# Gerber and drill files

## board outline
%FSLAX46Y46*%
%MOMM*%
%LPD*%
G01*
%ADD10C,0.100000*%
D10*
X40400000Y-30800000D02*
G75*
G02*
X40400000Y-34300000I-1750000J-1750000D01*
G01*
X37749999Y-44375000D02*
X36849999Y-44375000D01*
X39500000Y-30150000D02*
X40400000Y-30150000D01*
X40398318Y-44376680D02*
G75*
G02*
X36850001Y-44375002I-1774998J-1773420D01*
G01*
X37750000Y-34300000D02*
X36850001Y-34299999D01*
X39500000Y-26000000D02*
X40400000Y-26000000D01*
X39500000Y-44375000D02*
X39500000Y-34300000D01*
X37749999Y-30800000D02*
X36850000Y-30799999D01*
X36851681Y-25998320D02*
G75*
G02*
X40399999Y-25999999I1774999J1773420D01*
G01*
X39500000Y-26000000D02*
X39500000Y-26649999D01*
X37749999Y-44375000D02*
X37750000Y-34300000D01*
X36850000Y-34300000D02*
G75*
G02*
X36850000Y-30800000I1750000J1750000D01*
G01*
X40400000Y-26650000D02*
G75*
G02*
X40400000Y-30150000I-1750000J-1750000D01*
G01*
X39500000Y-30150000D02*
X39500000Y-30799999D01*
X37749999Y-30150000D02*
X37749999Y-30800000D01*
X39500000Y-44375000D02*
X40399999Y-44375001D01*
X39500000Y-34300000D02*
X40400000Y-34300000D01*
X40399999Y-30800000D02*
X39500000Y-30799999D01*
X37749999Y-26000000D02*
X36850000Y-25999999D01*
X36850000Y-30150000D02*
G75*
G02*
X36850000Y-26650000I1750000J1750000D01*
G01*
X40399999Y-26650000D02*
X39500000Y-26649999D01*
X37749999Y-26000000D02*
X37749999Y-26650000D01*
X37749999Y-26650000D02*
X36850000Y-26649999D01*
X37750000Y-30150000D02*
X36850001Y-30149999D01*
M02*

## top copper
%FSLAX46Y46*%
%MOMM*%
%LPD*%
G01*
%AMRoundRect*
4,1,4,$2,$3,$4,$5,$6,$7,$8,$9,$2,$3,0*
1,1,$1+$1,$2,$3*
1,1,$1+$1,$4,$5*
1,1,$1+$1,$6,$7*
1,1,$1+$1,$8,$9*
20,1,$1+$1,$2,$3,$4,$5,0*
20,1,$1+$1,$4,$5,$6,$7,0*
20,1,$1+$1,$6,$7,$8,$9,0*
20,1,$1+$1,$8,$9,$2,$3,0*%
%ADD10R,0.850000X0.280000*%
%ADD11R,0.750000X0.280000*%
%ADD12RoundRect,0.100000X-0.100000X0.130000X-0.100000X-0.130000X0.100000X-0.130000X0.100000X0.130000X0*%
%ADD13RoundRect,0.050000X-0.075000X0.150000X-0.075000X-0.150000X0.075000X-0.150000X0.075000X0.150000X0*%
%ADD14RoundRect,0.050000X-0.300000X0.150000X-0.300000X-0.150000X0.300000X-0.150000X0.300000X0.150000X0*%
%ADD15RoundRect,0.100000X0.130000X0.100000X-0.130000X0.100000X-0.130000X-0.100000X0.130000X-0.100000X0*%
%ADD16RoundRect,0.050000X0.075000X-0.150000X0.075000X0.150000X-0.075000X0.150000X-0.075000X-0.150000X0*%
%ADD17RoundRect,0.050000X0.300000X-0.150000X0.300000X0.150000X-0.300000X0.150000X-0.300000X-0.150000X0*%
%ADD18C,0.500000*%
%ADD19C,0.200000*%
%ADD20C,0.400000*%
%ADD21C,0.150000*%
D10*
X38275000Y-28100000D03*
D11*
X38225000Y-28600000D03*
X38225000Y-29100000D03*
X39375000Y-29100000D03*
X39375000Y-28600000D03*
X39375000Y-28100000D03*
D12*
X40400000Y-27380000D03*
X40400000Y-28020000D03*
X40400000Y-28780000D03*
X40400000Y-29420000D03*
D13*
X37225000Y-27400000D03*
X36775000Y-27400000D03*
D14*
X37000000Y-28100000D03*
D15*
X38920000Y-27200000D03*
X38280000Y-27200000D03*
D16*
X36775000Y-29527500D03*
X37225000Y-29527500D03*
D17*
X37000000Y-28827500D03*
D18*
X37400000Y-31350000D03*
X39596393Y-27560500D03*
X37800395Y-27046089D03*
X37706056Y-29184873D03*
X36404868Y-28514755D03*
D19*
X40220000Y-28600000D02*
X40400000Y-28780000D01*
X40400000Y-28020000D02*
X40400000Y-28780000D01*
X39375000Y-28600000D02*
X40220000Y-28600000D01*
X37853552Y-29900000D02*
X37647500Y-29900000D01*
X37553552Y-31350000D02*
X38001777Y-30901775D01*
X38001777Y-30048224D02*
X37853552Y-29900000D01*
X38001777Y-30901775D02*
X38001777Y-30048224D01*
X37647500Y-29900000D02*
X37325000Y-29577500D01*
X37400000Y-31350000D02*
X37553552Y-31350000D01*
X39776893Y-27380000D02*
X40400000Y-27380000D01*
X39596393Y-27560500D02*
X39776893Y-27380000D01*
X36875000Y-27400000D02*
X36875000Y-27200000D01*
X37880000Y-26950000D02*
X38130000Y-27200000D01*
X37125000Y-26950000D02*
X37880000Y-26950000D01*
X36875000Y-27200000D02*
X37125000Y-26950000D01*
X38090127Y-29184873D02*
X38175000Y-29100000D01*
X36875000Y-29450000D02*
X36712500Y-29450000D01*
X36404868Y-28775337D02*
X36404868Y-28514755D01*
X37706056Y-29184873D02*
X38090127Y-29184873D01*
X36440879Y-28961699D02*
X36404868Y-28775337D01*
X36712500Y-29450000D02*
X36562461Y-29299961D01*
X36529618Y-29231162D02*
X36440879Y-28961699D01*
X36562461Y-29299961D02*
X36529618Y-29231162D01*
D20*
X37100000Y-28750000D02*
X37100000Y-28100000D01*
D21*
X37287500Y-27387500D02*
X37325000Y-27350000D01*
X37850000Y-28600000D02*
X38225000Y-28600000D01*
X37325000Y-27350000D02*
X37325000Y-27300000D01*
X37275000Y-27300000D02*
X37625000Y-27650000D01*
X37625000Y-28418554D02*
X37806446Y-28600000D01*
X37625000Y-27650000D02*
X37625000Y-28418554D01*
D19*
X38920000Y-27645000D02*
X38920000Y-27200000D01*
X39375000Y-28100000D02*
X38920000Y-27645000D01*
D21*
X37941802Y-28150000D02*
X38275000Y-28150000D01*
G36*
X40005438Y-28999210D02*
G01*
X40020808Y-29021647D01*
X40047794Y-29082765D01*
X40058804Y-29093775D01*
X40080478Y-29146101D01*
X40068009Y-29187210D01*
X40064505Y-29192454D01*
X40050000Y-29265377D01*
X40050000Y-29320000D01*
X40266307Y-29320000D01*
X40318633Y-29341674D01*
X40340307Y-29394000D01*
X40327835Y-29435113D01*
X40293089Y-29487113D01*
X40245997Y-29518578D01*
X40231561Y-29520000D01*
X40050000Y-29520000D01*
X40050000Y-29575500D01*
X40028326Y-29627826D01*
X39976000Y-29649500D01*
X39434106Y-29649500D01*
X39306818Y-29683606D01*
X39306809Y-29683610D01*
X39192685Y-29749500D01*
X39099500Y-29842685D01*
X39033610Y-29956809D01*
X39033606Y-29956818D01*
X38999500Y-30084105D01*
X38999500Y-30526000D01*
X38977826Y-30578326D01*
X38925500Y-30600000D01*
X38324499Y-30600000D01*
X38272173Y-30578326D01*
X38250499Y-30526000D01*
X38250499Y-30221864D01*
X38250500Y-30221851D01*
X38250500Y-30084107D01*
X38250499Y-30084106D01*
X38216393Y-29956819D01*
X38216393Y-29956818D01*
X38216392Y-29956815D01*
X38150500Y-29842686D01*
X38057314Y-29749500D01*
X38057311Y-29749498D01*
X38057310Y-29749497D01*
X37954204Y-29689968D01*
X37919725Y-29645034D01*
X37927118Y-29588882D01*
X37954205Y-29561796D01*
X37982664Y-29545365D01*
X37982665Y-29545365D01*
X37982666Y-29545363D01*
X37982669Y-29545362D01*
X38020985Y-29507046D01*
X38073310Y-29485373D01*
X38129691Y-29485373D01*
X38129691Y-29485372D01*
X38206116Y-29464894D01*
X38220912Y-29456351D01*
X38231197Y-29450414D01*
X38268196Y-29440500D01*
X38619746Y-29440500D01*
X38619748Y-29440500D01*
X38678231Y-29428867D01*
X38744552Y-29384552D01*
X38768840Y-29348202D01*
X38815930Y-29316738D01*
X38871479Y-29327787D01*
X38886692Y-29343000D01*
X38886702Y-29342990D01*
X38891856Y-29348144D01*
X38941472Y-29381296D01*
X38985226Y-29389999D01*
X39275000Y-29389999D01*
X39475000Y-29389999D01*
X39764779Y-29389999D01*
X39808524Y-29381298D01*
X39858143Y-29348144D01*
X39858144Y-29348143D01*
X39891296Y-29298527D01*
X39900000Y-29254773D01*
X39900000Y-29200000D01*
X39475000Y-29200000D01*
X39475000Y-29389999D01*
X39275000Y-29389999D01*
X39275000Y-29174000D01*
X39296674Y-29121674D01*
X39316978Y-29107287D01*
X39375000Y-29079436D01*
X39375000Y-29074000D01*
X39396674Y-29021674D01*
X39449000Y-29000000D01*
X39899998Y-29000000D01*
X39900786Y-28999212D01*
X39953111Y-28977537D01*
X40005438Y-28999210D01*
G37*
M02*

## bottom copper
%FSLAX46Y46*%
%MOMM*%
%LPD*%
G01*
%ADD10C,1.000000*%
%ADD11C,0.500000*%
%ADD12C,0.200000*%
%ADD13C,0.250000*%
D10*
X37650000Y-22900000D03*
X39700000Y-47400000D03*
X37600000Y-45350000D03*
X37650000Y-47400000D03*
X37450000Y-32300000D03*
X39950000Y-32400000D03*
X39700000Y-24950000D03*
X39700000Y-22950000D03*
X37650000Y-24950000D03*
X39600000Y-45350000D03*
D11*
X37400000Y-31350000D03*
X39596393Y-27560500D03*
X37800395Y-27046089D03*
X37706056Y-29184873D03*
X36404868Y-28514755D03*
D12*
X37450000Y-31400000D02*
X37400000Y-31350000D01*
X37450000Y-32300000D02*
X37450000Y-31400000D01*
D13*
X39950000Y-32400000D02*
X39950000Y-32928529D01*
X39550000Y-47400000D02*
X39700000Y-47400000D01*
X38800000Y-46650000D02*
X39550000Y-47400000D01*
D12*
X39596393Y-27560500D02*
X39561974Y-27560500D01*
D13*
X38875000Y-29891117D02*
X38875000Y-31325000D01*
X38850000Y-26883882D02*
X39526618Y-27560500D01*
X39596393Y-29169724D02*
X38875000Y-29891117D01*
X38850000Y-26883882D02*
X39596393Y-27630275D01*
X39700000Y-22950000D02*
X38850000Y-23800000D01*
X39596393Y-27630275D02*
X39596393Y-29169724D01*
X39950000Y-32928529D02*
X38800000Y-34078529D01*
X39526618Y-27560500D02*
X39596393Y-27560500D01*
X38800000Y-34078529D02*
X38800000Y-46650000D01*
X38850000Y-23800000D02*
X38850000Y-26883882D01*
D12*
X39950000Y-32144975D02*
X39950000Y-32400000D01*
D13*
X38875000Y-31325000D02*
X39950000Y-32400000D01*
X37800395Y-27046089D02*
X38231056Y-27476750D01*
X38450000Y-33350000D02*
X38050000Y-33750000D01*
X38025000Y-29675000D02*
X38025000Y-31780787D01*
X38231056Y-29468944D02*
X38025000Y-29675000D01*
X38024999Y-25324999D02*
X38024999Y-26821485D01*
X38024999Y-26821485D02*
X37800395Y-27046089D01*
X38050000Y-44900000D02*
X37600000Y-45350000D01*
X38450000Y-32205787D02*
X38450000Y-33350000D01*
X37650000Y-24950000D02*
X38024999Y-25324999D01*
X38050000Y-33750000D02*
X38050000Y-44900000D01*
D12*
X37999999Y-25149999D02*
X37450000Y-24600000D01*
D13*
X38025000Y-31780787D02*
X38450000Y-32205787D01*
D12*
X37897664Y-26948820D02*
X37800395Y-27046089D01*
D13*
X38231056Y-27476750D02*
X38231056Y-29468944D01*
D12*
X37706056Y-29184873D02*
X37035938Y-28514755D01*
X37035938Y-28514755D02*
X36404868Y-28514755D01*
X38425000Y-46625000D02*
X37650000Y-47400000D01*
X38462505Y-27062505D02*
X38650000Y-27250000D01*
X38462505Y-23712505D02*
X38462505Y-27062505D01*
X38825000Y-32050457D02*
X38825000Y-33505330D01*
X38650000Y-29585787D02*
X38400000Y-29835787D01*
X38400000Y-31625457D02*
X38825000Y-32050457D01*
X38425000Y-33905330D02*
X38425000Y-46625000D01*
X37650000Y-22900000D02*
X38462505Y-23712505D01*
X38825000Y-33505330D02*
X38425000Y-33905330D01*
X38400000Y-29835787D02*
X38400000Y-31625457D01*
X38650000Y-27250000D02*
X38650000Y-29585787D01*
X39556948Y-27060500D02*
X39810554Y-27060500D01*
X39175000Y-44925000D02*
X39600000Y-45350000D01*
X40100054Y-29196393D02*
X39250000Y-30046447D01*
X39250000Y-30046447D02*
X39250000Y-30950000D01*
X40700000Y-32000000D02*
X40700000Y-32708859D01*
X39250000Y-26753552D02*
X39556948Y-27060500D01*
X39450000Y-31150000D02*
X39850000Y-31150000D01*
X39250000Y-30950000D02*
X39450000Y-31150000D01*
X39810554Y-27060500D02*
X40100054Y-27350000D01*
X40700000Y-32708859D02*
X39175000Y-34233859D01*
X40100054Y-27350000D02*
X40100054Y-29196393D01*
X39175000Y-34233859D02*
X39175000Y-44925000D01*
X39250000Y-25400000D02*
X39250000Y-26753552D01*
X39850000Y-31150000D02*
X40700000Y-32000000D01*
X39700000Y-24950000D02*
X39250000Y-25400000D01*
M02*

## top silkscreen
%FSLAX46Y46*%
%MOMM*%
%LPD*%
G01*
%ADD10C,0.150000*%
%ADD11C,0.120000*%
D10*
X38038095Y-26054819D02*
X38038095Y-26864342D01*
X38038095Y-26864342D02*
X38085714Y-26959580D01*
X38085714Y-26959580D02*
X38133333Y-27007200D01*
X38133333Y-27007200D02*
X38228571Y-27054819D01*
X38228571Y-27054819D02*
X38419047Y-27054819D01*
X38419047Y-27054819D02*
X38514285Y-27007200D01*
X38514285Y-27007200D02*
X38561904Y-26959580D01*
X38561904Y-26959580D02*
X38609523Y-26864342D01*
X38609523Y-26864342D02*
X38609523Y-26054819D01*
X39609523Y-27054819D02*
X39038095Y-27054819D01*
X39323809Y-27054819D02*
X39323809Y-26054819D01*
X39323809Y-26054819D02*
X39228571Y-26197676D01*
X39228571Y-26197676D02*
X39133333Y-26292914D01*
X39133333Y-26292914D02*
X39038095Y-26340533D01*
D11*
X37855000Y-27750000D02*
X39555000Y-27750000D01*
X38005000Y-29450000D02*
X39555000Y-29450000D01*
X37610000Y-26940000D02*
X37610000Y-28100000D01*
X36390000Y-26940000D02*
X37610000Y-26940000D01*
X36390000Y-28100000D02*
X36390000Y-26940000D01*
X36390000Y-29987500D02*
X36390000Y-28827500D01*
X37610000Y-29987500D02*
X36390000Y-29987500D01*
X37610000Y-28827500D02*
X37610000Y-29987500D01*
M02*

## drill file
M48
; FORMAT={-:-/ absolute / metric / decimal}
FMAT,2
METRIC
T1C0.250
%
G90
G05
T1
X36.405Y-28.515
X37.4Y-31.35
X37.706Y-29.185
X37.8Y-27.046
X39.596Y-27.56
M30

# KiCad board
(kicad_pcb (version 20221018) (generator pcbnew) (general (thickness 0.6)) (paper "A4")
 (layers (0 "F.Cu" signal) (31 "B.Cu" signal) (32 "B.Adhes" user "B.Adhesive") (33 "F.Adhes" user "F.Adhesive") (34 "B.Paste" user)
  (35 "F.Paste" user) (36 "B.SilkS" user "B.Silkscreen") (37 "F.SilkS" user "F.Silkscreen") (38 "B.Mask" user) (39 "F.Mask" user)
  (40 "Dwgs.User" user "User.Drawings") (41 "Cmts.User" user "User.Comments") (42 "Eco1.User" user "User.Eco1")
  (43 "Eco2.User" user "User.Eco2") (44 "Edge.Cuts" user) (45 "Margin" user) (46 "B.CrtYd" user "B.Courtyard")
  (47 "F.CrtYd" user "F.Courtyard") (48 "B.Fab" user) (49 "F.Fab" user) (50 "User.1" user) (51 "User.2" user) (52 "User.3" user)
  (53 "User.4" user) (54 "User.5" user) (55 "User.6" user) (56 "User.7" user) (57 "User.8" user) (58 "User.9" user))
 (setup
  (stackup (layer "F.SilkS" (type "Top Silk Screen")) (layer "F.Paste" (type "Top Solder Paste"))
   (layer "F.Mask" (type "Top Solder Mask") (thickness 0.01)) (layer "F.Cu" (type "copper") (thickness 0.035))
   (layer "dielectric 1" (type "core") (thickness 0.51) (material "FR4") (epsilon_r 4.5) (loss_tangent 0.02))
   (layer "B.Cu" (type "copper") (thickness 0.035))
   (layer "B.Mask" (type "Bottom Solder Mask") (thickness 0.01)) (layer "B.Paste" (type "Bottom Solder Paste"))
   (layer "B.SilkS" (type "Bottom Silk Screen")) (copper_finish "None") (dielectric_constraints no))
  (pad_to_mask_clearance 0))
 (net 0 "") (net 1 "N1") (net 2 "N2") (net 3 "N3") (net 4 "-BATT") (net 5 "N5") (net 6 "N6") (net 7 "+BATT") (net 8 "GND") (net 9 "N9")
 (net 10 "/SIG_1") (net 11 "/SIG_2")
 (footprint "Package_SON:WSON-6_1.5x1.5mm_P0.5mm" (layer "F.Cu") (at 38.8 28.6)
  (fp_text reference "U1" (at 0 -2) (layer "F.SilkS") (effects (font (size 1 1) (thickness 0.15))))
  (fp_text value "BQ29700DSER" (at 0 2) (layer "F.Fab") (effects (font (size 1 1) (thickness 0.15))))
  (fp_line (start -0.945 -0.85) (end 0.755 -0.85) (stroke (width 0.12) (type solid)) (layer "F.SilkS"))
  (fp_line (start -0.795 0.85) (end 0.755 0.85) (stroke (width 0.12) (type solid)) (layer "F.SilkS"))
  (pad "1" smd rect (at -0.525 -0.5 270) (size 0.28 0.85) (layers "F.Cu" "F.Paste" "F.Mask") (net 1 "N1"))
  (pad "2" smd rect (at -0.575 0 270) (size 0.28 0.75) (layers "F.Cu" "F.Paste" "F.Mask") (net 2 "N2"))
  (pad "3" smd rect (at -0.575 0.5 270) (size 0.28 0.75) (layers "F.Cu" "F.Paste" "F.Mask") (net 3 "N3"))
  (pad "4" smd rect (at 0.575 0.5 270) (size 0.28 0.75) (layers "F.Cu" "F.Paste" "F.Mask") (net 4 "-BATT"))
  (pad "5" smd rect (at 0.575 0 270) (size 0.28 0.75) (layers "F.Cu" "F.Paste" "F.Mask") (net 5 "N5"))
  (pad "6" smd rect (at 0.575 -0.5 270) (size 0.28 0.75) (layers "F.Cu" "F.Paste" "F.Mask") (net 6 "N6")))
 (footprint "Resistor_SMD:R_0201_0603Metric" (layer "F.Cu") (at 40.4 27.7 -90)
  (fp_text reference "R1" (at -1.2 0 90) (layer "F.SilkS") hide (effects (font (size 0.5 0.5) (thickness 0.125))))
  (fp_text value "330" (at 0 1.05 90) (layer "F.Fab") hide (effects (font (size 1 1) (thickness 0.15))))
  (pad "" smd roundrect (at -0.345 0 270) (size 0.318 0.36) (layers "F.Paste") (roundrect_rratio 0.25))
  (pad "" smd roundrect (at 0.345 0 270) (size 0.318 0.36) (layers "F.Paste") (roundrect_rratio 0.25))
  (pad "1" smd roundrect (at -0.32 0 270) (size 0.46 0.4) (layers "F.Cu" "F.Mask") (roundrect_rratio 0.25) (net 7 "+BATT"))
  (pad "2" smd roundrect (at 0.32 0 270) (size 0.46 0.4) (layers "F.Cu" "F.Mask") (roundrect_rratio 0.25) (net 5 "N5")))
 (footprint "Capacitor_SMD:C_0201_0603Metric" (layer "F.Cu") (at 40.4 29.1 -90)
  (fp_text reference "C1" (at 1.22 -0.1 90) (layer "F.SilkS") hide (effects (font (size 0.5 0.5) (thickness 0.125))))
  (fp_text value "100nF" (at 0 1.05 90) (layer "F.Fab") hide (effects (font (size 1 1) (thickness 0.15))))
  (pad "" smd roundrect (at -0.345 0 270) (size 0.318 0.36) (layers "F.Paste") (roundrect_rratio 0.25))
  (pad "" smd roundrect (at 0.345 0 270) (size 0.318 0.36) (layers "F.Paste") (roundrect_rratio 0.25))
  (pad "1" smd roundrect (at -0.32 0 270) (size 0.46 0.4) (layers "F.Cu" "F.Mask") (roundrect_rratio 0.25) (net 5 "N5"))
  (pad "2" smd roundrect (at 0.32 0 270) (size 0.46 0.4) (layers "F.Cu" "F.Mask") (roundrect_rratio 0.25) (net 4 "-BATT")))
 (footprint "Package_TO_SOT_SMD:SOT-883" (layer "F.Cu") (at 37 27.75 -90)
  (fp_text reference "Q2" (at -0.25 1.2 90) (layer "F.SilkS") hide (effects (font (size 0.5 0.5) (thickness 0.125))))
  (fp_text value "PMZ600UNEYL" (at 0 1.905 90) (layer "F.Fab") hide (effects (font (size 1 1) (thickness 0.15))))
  (fp_line (start -0.81 -0.61) (end 0.35 -0.61) (stroke (width 0.12) (type solid)) (layer "F.SilkS"))
  (fp_line (start -0.81 0.61) (end -0.81 -0.61) (stroke (width 0.12) (type solid)) (layer "F.SilkS"))
  (fp_line (start 0.35 0.61) (end -0.81 0.61) (stroke (width 0.12) (type solid)) (layer "F.SilkS"))
  (pad "1" smd roundrect (at -0.35 -0.225 270) (size 0.4 0.25) (layers "F.Cu" "F.Paste" "F.Mask") (roundrect_rratio 0.2) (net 2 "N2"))
  (pad "2" smd roundrect (at -0.35 0.225 270) (size 0.4 0.25) (layers "F.Cu" "F.Paste" "F.Mask") (roundrect_rratio 0.2) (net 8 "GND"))
  (pad "3" smd roundrect (at 0.35 0 270) (size 0.4 0.7) (layers "F.Cu" "F.Paste" "F.Mask") (roundrect_rratio 0.125) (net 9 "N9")))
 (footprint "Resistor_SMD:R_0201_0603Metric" (layer "F.Cu") (at 38.6 27.2 180)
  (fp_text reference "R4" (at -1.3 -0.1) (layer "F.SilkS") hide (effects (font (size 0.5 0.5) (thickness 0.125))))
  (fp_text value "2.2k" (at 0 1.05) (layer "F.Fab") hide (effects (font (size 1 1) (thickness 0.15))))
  (pad "" smd roundrect (at -0.345 0 180) (size 0.318 0.36) (layers "F.Paste") (roundrect_rratio 0.25))
  (pad "" smd roundrect (at 0.345 0 180) (size 0.318 0.36) (layers "F.Paste") (roundrect_rratio 0.25))
  (pad "1" smd roundrect (at -0.32 0 180) (size 0.46 0.4) (layers "F.Cu" "F.Mask") (roundrect_rratio 0.25) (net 6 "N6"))
  (pad "2" smd roundrect (at 0.32 0 180) (size 0.46 0.4) (layers "F.Cu" "F.Mask") (roundrect_rratio 0.25) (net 8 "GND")))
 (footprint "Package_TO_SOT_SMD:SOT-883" (layer "F.Cu") (at 37 29.1775 90)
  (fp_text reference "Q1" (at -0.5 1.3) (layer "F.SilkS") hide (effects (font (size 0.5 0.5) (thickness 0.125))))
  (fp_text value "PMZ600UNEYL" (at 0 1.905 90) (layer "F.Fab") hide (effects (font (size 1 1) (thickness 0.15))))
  (fp_line (start -0.81 -0.61) (end 0.35 -0.61) (stroke (width 0.12) (type solid)) (layer "F.SilkS"))
  (fp_line (start -0.81 0.61) (end -0.81 -0.61) (stroke (width 0.12) (type solid)) (layer "F.SilkS"))
  (fp_line (start 0.35 0.61) (end -0.81 0.61) (stroke (width 0.12) (type solid)) (layer "F.SilkS"))
  (pad "1" smd roundrect (at -0.35 -0.225 90) (size 0.4 0.25) (layers "F.Cu" "F.Paste" "F.Mask") (roundrect_rratio 0.2) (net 3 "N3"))
  (pad "2" smd roundrect (at -0.35 0.225 90) (size 0.4 0.25) (layers "F.Cu" "F.Paste" "F.Mask") (roundrect_rratio 0.2) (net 4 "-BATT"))
  (pad "3" smd roundrect (at 0.35 0 90) (size 0.4 0.7) (layers "F.Cu" "F.Paste" "F.Mask") (roundrect_rratio 0.125) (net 9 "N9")))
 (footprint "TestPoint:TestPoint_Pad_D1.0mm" (layer "B.Cu") (at 37.65 22.9 180)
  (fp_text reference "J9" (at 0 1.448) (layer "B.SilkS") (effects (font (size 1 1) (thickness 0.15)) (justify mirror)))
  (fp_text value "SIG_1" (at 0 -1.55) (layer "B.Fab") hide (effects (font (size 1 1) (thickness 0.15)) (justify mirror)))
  (pad "1" smd circle (at 0 0 180) (size 1 1) (layers "B.Cu" "B.Mask") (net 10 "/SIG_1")))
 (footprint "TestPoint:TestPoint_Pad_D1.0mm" (layer "B.Cu") (at 39.7 47.4 180)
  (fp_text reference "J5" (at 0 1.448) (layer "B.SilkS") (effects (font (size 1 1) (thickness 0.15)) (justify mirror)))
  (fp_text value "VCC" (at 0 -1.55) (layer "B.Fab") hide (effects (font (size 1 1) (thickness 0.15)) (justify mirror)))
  (pad "1" smd circle (at 0 0 180) (size 1 1) (layers "B.Cu" "B.Mask") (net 7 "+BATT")))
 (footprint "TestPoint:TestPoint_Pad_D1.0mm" (layer "B.Cu") (at 37.6 45.35 180)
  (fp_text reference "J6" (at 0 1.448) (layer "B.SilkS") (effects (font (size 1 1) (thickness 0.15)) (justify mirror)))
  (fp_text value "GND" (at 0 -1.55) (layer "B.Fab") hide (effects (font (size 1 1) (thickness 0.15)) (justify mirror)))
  (pad "1" smd circle (at 0 0 180) (size 1 1) (layers "B.Cu" "B.Mask") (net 8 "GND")))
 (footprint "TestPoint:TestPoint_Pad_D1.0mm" (layer "B.Cu") (at 37.65 47.4 180)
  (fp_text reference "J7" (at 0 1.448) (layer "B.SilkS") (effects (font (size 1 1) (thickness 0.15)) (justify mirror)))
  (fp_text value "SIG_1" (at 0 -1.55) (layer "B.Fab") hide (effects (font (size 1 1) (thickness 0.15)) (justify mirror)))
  (pad "1" smd circle (at 0 0 180) (size 1 1) (layers "B.Cu" "B.Mask") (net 10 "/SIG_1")))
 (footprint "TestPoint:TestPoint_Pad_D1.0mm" (layer "B.Cu") (at 37.45 32.3 90)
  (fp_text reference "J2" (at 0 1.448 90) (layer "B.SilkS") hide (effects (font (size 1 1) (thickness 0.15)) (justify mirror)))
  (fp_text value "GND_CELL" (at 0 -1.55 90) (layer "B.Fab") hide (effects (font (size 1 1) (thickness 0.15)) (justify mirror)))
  (pad "1" smd circle (at 0 0 90) (size 1 1) (layers "B.Cu" "B.Mask") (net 4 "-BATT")))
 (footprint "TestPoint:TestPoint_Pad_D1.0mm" (layer "B.Cu") (at 39.95 32.4 90)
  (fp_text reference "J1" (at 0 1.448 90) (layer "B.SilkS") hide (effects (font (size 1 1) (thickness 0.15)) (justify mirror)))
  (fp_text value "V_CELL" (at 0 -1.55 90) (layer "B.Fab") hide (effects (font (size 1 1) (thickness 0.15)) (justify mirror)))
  (pad "1" smd circle (at 0 0 90) (size 1 1) (layers "B.Cu" "B.Mask") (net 7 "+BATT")))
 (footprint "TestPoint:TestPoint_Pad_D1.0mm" (layer "B.Cu") (at 39.7 24.95 180)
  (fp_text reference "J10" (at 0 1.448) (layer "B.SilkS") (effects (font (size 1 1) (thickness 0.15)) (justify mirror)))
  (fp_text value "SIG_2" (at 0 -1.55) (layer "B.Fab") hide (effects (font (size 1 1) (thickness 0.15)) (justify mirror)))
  (pad "1" smd circle (at 0 0 180) (size 1 1) (layers "B.Cu" "B.Mask") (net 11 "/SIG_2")))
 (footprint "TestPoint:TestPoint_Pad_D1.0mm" (layer "B.Cu") (at 39.7 22.95 180)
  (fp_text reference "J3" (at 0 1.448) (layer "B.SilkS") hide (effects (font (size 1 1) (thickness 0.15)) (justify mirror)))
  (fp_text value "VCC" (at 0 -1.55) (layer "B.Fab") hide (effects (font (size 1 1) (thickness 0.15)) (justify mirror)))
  (pad "1" smd circle (at 0 0 180) (size 1 1) (layers "B.Cu" "B.Mask") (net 7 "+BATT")))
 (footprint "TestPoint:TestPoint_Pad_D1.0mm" (layer "B.Cu") (at 37.65 24.95 180)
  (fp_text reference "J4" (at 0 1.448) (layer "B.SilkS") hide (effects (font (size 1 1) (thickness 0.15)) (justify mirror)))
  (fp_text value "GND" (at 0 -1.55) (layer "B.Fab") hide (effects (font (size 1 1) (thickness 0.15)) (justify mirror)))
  (pad "1" smd circle (at 0 0 180) (size 1 1) (layers "B.Cu" "B.Mask") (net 8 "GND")))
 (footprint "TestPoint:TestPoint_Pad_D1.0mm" (layer "B.Cu") (at 39.6 45.35 180)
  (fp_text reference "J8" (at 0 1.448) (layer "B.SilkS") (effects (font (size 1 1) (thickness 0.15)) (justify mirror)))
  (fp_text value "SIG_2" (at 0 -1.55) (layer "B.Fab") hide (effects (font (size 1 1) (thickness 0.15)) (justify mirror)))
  (pad "1" smd circle (at 0 0 180) (size 1 1) (layers "B.Cu" "B.Mask") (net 11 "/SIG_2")))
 (gr_arc (start 40.4 30.8) (mid 41.124874 32.550001) (end 40.4 34.300001) (stroke (width 0.1) (type default)) (layer "Edge.Cuts"))
 (gr_line (start 37.749999 44.375) (end 36.849999 44.375) (stroke (width 0.1) (type default)) (layer "Edge.Cuts"))
 (gr_line (start 39.5 30.15) (end 40.4 30.15) (stroke (width 0.1) (type default)) (layer "Edge.Cuts"))
 (gr_arc (start 40.398318 44.37668) (mid 38.622131 48.659208) (end 36.85 44.375001) (stroke (width 0.1) (type default)) (layer "Edge.Cuts"))
 (gr_line (start 37.75 34.3) (end 36.850001 34.299999) (stroke (width 0.1) (type default)) (layer "Edge.Cuts"))
 (gr_line (start 39.5 26) (end 40.4 26) (stroke (width 0.1) (type default)) (layer "Edge.Cuts"))
 (gr_line (start 39.5 44.375) (end 39.5 34.3) (stroke (width 0.1) (type default)) (layer "Edge.Cuts"))
 (gr_line (start 37.749999 30.8) (end 36.85 30.799999) (stroke (width 0.1) (type default)) (layer "Edge.Cuts"))
 (gr_arc (start 36.851681 25.99832) (mid 38.627868 21.715792) (end 40.399999 25.999999) (stroke (width 0.1) (type default))
  (layer "Edge.Cuts"))
 (gr_line (start 39.5 26) (end 39.5 26.649999) (stroke (width 0.1) (type default)) (layer "Edge.Cuts"))
 (gr_line (start 37.749999 44.375) (end 37.75 34.3) (stroke (width 0.1) (type default)) (layer "Edge.Cuts"))
 (gr_arc (start 36.85 34.3) (mid 36.125126 32.55) (end 36.85 30.799999) (stroke (width 0.1) (type default)) (layer "Edge.Cuts"))
 (gr_arc (start 40.4 26.65) (mid 41.124874 28.4) (end 40.4 30.150001) (stroke (width 0.1) (type default)) (layer "Edge.Cuts"))
 (gr_line (start 39.5 30.15) (end 39.5 30.799999) (stroke (width 0.1) (type default)) (layer "Edge.Cuts"))
 (gr_line (start 37.749999 30.15) (end 37.749999 30.8) (stroke (width 0.1) (type default)) (layer "Edge.Cuts"))
 (gr_line (start 39.5 44.375) (end 40.399999 44.375001) (stroke (width 0.1) (type default)) (layer "Edge.Cuts"))
 (gr_line (start 39.5 34.3) (end 40.4 34.3) (stroke (width 0.1) (type default)) (layer "Edge.Cuts"))
 (gr_line (start 40.399999 30.8) (end 39.5 30.799999) (stroke (width 0.1) (type default)) (layer "Edge.Cuts"))
 (gr_line (start 37.749999 26) (end 36.85 25.999999) (stroke (width 0.1) (type default)) (layer "Edge.Cuts"))
 (gr_arc (start 36.85 30.15) (mid 36.125126 28.4) (end 36.85 26.649999) (stroke (width 0.1) (type default)) (layer "Edge.Cuts"))
 (gr_line (start 40.399999 26.65) (end 39.5 26.649999) (stroke (width 0.1) (type default)) (layer "Edge.Cuts"))
 (gr_line (start 37.749999 26) (end 37.749999 26.65) (stroke (width 0.1) (type default)) (layer "Edge.Cuts"))
 (gr_line (start 37.749999 26.65) (end 36.85 26.649999) (stroke (width 0.1) (type default)) (layer "Edge.Cuts"))
 (gr_line (start 37.75 30.15) (end 36.850001 30.149999) (stroke (width 0.1) (type default)) (layer "Edge.Cuts"))
 (segment (start 40.22 28.6) (end 40.4 28.78) (width 0.2) (layer "F.Cu") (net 5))
 (segment (start 40.4 28.02) (end 40.4 28.78) (width 0.2) (layer "F.Cu") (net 5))
 (segment (start 39.375 28.6) (end 40.22 28.6) (width 0.2) (layer "F.Cu") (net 5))
 (segment (start 37.853552 29.9) (end 37.6475 29.9) (width 0.2) (layer "F.Cu") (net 4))
 (segment (start 37.553552 31.35) (end 38.001777 30.901775) (width 0.2) (layer "F.Cu") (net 4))
 (segment (start 38.001777 30.048224) (end 37.853552 29.9) (width 0.2) (layer "F.Cu") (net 4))
 (segment (start 38.001777 30.901775) (end 38.001777 30.048224) (width 0.2) (layer "F.Cu") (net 4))
 (segment (start 37.6475 29.9) (end 37.325 29.5775) (width 0.2) (layer "F.Cu") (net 4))
 (segment (start 37.4 31.35) (end 37.553552 31.35) (width 0.2) (layer "F.Cu") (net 4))
 (via (at 37.4 31.35) (size 0.5) (drill 0.25) (layers "F.Cu" "B.Cu") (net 4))
 (segment (start 37.45 31.4) (end 37.4 31.35) (width 0.2) (layer "B.Cu") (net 4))
 (segment (start 37.45 32.3) (end 37.45 31.4) (width 0.2) (layer "B.Cu") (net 4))
 (segment (start 39.776893 27.38) (end 40.4 27.38) (width 0.2) (layer "F.Cu") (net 7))
 (segment (start 39.596393 27.5605) (end 39.776893 27.38) (width 0.2) (layer "F.Cu") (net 7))
 (via (at 39.596393 27.5605) (size 0.5) (drill 0.25) (layers "F.Cu" "B.Cu") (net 7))
 (segment (start 39.95 32.4) (end 39.95 32.928529) (width 0.25) (layer "B.Cu") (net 7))
 (segment (start 39.55 47.4) (end 39.7 47.4) (width 0.25) (layer "B.Cu") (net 7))
 (segment (start 38.8 46.65) (end 39.55 47.4) (width 0.25) (layer "B.Cu") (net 7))
 (segment (start 39.596393 27.5605) (end 39.561974 27.5605) (width 0.2) (layer "B.Cu") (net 7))
 (segment (start 38.875 29.891117) (end 38.875 31.325) (width 0.25) (layer "B.Cu") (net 7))
 (segment (start 38.85 26.883882) (end 39.526618 27.5605) (width 0.25) (layer "B.Cu") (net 7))
 (segment (start 39.596393 29.169724) (end 38.875 29.891117) (width 0.25) (layer "B.Cu") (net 7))
 (segment (start 38.85 26.883882) (end 39.596393 27.630275) (width 0.25) (layer "B.Cu") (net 7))
 (segment (start 39.7 22.95) (end 38.85 23.8) (width 0.25) (layer "B.Cu") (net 7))
 (segment (start 39.596393 27.630275) (end 39.596393 29.169724) (width 0.25) (layer "B.Cu") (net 7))
 (segment (start 39.95 32.928529) (end 38.8 34.078529) (width 0.25) (layer "B.Cu") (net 7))
 (segment (start 39.526618 27.5605) (end 39.596393 27.5605) (width 0.25) (layer "B.Cu") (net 7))
 (segment (start 38.8 34.078529) (end 38.8 46.65) (width 0.25) (layer "B.Cu") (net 7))
 (segment (start 38.85 23.8) (end 38.85 26.883882) (width 0.25) (layer "B.Cu") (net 7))
 (segment (start 39.95 32.144975) (end 39.95 32.4) (width 0.2) (layer "B.Cu") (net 7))
 (segment (start 38.875 31.325) (end 39.95 32.4) (width 0.25) (layer "B.Cu") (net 7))
 (segment (start 36.875 27.4) (end 36.875 27.2) (width 0.2) (layer "F.Cu") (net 8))
 (segment (start 37.88 26.95) (end 38.13 27.2) (width 0.2) (layer "F.Cu") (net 8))
 (segment (start 37.125 26.95) (end 37.88 26.95) (width 0.2) (layer "F.Cu") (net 8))
 (segment (start 36.875 27.2) (end 37.125 26.95) (width 0.2) (layer "F.Cu") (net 8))
 (via (at 37.800395 27.046089) (size 0.5) (drill 0.25) (layers "F.Cu" "B.Cu") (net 8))
 (segment (start 37.800395 27.046089) (end 38.231056 27.47675) (width 0.25) (layer "B.Cu") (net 8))
 (segment (start 38.45 33.35) (end 38.05 33.75) (width 0.25) (layer "B.Cu") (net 8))
 (segment (start 38.025 29.675) (end 38.025 31.780787) (width 0.25) (layer "B.Cu") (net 8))
 (segment (start 38.231056 29.468944) (end 38.025 29.675) (width 0.25) (layer "B.Cu") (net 8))
 (segment (start 38.024999 25.324999) (end 38.024999 26.821485) (width 0.25) (layer "B.Cu") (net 8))
 (segment (start 38.024999 26.821485) (end 37.800395 27.046089) (width 0.25) (layer "B.Cu") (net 8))
 (segment (start 38.05 44.9) (end 37.6 45.35) (width 0.25) (layer "B.Cu") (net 8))
 (segment (start 38.45 32.205787) (end 38.45 33.35) (width 0.25) (layer "B.Cu") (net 8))
 (segment (start 37.65 24.95) (end 38.024999 25.324999) (width 0.25) (layer "B.Cu") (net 8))
 (segment (start 38.05 33.75) (end 38.05 44.9) (width 0.25) (layer "B.Cu") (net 8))
 (segment (start 37.999999 25.149999) (end 37.45 24.6) (width 0.2) (layer "B.Cu") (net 8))
 (segment (start 38.025 31.780787) (end 38.45 32.205787) (width 0.25) (layer "B.Cu") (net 8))
 (segment (start 37.897664 26.94882) (end 37.800395 27.046089) (width 0.2) (layer "B.Cu") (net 8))
 (segment (start 38.231056 27.47675) (end 38.231056 29.468944) (width 0.25) (layer "B.Cu") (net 8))
 (segment (start 38.090127 29.184873) (end 38.175 29.1) (width 0.2) (layer "F.Cu") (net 3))
 (segment (start 36.875 29.45) (end 36.7125 29.45) (width 0.2) (layer "F.Cu") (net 3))
 (segment (start 36.404868 28.775337) (end 36.404868 28.514755) (width 0.2) (layer "F.Cu") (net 3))
 (segment (start 37.706056 29.184873) (end 38.090127 29.184873) (width 0.2) (layer "F.Cu") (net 3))
 (segment (start 36.440879 28.961699) (end 36.404868 28.775337) (width 0.2) (layer "F.Cu") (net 3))
 (segment (start 36.7125 29.45) (end 36.562461 29.299961) (width 0.2) (layer "F.Cu") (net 3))
 (segment (start 36.529618 29.231162) (end 36.440879 28.961699) (width 0.2) (layer "F.Cu") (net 3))
 (segment (start 36.562461 29.299961) (end 36.529618 29.231162) (width 0.2) (layer "F.Cu") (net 3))
 (via (at 37.706056 29.184873) (size 0.5) (drill 0.25) (layers "F.Cu" "B.Cu") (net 3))
 (via (at 36.404868 28.514755) (size 0.5) (drill 0.25) (layers "F.Cu" "B.Cu") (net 3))
 (segment (start 37.706056 29.184873) (end 37.035938 28.514755) (width 0.2) (layer "B.Cu") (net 3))
 (segment (start 37.035938 28.514755) (end 36.404868 28.514755) (width 0.2) (layer "B.Cu") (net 3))
 (segment (start 37.1 28.75) (end 37.1 28.1) (width 0.4) (layer "F.Cu") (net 9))
 (segment (start 37.2875 27.3875) (end 37.325 27.35) (width 0.15) (layer "F.Cu") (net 2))
 (segment (start 37.85 28.6) (end 38.225 28.6) (width 0.15) (layer "F.Cu") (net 2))
 (segment (start 37.325 27.35) (end 37.325 27.3) (width 0.15) (layer "F.Cu") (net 2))
 (segment (start 37.275 27.3) (end 37.625 27.65) (width 0.15) (layer "F.Cu") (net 2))
 (segment (start 37.625 28.418554) (end 37.806446 28.6) (width 0.15) (layer "F.Cu") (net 2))
 (segment (start 37.625 27.65) (end 37.625 28.418554) (width 0.15) (layer "F.Cu") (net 2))
 (segment (start 38.92 27.645) (end 38.92 27.2) (width 0.2) (layer "F.Cu") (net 6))
 (segment (start 39.375 28.1) (end 38.92 27.645) (width 0.2) (layer "F.Cu") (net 6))
 (segment (start 37.941802 28.15) (end 38.275 28.15) (width 0.15) (layer "F.Cu") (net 1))
 (segment (start 38.425 46.625) (end 37.65 47.4) (width 0.2) (layer "B.Cu") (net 10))
 (segment (start 38.462505 27.062505) (end 38.65 27.25) (width 0.2) (layer "B.Cu") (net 10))
 (segment (start 38.462505 23.712505) (end 38.462505 27.062505) (width 0.2) (layer "B.Cu") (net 10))
 (segment (start 38.825 32.050457) (end 38.825 33.50533) (width 0.2) (layer "B.Cu") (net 10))
 (segment (start 38.65 29.585787) (end 38.4 29.835787) (width 0.2) (layer "B.Cu") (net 10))
 (segment (start 38.4 31.625457) (end 38.825 32.050457) (width 0.2) (layer "B.Cu") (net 10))
 (segment (start 38.425 33.90533) (end 38.425 46.625) (width 0.2) (layer "B.Cu") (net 10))
 (segment (start 37.65 22.9) (end 38.462505 23.712505) (width 0.2) (layer "B.Cu") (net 10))
 (segment (start 38.825 33.50533) (end 38.425 33.90533) (width 0.2) (layer "B.Cu") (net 10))
 (segment (start 38.4 29.835787) (end 38.4 31.625457) (width 0.2) (layer "B.Cu") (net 10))
 (segment (start 38.65 27.25) (end 38.65 29.585787) (width 0.2) (layer "B.Cu") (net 10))
 (segment (start 39.556948 27.0605) (end 39.810554 27.0605) (width 0.2) (layer "B.Cu") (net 11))
 (segment (start 39.175 44.925) (end 39.6 45.35) (width 0.2) (layer "B.Cu") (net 11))
 (segment (start 40.100054 29.196393) (end 39.25 30.046447) (width 0.2) (layer "B.Cu") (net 11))
 (segment (start 39.25 30.046447) (end 39.25 30.95) (width 0.2) (layer "B.Cu") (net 11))
 (segment (start 40.7 32) (end 40.7 32.708859) (width 0.2) (layer "B.Cu") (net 11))
 (segment (start 39.25 26.753552) (end 39.556948 27.0605) (width 0.2) (layer "B.Cu") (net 11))
 (segment (start 39.45 31.15) (end 39.85 31.15) (width 0.2) (layer "B.Cu") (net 11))
 (segment (start 39.25 30.95) (end 39.45 31.15) (width 0.2) (layer "B.Cu") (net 11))
 (segment (start 39.810554 27.0605) (end 40.100054 27.35) (width 0.2) (layer "B.Cu") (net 11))
 (segment (start 40.7 32.708859) (end 39.175 34.233859) (width 0.2) (layer "B.Cu") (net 11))
 (segment (start 40.100054 27.35) (end 40.100054 29.196393) (width 0.2) (layer "B.Cu") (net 11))
 (segment (start 39.175 34.233859) (end 39.175 44.925) (width 0.2) (layer "B.Cu") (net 11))
 (segment (start 39.25 25.4) (end 39.25 26.753552) (width 0.2) (layer "B.Cu") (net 11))
 (segment (start 39.85 31.15) (end 40.7 32) (width 0.2) (layer "B.Cu") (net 11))
 (segment (start 39.7 24.95) (end 39.25 25.4) (width 0.2) (layer "B.Cu") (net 11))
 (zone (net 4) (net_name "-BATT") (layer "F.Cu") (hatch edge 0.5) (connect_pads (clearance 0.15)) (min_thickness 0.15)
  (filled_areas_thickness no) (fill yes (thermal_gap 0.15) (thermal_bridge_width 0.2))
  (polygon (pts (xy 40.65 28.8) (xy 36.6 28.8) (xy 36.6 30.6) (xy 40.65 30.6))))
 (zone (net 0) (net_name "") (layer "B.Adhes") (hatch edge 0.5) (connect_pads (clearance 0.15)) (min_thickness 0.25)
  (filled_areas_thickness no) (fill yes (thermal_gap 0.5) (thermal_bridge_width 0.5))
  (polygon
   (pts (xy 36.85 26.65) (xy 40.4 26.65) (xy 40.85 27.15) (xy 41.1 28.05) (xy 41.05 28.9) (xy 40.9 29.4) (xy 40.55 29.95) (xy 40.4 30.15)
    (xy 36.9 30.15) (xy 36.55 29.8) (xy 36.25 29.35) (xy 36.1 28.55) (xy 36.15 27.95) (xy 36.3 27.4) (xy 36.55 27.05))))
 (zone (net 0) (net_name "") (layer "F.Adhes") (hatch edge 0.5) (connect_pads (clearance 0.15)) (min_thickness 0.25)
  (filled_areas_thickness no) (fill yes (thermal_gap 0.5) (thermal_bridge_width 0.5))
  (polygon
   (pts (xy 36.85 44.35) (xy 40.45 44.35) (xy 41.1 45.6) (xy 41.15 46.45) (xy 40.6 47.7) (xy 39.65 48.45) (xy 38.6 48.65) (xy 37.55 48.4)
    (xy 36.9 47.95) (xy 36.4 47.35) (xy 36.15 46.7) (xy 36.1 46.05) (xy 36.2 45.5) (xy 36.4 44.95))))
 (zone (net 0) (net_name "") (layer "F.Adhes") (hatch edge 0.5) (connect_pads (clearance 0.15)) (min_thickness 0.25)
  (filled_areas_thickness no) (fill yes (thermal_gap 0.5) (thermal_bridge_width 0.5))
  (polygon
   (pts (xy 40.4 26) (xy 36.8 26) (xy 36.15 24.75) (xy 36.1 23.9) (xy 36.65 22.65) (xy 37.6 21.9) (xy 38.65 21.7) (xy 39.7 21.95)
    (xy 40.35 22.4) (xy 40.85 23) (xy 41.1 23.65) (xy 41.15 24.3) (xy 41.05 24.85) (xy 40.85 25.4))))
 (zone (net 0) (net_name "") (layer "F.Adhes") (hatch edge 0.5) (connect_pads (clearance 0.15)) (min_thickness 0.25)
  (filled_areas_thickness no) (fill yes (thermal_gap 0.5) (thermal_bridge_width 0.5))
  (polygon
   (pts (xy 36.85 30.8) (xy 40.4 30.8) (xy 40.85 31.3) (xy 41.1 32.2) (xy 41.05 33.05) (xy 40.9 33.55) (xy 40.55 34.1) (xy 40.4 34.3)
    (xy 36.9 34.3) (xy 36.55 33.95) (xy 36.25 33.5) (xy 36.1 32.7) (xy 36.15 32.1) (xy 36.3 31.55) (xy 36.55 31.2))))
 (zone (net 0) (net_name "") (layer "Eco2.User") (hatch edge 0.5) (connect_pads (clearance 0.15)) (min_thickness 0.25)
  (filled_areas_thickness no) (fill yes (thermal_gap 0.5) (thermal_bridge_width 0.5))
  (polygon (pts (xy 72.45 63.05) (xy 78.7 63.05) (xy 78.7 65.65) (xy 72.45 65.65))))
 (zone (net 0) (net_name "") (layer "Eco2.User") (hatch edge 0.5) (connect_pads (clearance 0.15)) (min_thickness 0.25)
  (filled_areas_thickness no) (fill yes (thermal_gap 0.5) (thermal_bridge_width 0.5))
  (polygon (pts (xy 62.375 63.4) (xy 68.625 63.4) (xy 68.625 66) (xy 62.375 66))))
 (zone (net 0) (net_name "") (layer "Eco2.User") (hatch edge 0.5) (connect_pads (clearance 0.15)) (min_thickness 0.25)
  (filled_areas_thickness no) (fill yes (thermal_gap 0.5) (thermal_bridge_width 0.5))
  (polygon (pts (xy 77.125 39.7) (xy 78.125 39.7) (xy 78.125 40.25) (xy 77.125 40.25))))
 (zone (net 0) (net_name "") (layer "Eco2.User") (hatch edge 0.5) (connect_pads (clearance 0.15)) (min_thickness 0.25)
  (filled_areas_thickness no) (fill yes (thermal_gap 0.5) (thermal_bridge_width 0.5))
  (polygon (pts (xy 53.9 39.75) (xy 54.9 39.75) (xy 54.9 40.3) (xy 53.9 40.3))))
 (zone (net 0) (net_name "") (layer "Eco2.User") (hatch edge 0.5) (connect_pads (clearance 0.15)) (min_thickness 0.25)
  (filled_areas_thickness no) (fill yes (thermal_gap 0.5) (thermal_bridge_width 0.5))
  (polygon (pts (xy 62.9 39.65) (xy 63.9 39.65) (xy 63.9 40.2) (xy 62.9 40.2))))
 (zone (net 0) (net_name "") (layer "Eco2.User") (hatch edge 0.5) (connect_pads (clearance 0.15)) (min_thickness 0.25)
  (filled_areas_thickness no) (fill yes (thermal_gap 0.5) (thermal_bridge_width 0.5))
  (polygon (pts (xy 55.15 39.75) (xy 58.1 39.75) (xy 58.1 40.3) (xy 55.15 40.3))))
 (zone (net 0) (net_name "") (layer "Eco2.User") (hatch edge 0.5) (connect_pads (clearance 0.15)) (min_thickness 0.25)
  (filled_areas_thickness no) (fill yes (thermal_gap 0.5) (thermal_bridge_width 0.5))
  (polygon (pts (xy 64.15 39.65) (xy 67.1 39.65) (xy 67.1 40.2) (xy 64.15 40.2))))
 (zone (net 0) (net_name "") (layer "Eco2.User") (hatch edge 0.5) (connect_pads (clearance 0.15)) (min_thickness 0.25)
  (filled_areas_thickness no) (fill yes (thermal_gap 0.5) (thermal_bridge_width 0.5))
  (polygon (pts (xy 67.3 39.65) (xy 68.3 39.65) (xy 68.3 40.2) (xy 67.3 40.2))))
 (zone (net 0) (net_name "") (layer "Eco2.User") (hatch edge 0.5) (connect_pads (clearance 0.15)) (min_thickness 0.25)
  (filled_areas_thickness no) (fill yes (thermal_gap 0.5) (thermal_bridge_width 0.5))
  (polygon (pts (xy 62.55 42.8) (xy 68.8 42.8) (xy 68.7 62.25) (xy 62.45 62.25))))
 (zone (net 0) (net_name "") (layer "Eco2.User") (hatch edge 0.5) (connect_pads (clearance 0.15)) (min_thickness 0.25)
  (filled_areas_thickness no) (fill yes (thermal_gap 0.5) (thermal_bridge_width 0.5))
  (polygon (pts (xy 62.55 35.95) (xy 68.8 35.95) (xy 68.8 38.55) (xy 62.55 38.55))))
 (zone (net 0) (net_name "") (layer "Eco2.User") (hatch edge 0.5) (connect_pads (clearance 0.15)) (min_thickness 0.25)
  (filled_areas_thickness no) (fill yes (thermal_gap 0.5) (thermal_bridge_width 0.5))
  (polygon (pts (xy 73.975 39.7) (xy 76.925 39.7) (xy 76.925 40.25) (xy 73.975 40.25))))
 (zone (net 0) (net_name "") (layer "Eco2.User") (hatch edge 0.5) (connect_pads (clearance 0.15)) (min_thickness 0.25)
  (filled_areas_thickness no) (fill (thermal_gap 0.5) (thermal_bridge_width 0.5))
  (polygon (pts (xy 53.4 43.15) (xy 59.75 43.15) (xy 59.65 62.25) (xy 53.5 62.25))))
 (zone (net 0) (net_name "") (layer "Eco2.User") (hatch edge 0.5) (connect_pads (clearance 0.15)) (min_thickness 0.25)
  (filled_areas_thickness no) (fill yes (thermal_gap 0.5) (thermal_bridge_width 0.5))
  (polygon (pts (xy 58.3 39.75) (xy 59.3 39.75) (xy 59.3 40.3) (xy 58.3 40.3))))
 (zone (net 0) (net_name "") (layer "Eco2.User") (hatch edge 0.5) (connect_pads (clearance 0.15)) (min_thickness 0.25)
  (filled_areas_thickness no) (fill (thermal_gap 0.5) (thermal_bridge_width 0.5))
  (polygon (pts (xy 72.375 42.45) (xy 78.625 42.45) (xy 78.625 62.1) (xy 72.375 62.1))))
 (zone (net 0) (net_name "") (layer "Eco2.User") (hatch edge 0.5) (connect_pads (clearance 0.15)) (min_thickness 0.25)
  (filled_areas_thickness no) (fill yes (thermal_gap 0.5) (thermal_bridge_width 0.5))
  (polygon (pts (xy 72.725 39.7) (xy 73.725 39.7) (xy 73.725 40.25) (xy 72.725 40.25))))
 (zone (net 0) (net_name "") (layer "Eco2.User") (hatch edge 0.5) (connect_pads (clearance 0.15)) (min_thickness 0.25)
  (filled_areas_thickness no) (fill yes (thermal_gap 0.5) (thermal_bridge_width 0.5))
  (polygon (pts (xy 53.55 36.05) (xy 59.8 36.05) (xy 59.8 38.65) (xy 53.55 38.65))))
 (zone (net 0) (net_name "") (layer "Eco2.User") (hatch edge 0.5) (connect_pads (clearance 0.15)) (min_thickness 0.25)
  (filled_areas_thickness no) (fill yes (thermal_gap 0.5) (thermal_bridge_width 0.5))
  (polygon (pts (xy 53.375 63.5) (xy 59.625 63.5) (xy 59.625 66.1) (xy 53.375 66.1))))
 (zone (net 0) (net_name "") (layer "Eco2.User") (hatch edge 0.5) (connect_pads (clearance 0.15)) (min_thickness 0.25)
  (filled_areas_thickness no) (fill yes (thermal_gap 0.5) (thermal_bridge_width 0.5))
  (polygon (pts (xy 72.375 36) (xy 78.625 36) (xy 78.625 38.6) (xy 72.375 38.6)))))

